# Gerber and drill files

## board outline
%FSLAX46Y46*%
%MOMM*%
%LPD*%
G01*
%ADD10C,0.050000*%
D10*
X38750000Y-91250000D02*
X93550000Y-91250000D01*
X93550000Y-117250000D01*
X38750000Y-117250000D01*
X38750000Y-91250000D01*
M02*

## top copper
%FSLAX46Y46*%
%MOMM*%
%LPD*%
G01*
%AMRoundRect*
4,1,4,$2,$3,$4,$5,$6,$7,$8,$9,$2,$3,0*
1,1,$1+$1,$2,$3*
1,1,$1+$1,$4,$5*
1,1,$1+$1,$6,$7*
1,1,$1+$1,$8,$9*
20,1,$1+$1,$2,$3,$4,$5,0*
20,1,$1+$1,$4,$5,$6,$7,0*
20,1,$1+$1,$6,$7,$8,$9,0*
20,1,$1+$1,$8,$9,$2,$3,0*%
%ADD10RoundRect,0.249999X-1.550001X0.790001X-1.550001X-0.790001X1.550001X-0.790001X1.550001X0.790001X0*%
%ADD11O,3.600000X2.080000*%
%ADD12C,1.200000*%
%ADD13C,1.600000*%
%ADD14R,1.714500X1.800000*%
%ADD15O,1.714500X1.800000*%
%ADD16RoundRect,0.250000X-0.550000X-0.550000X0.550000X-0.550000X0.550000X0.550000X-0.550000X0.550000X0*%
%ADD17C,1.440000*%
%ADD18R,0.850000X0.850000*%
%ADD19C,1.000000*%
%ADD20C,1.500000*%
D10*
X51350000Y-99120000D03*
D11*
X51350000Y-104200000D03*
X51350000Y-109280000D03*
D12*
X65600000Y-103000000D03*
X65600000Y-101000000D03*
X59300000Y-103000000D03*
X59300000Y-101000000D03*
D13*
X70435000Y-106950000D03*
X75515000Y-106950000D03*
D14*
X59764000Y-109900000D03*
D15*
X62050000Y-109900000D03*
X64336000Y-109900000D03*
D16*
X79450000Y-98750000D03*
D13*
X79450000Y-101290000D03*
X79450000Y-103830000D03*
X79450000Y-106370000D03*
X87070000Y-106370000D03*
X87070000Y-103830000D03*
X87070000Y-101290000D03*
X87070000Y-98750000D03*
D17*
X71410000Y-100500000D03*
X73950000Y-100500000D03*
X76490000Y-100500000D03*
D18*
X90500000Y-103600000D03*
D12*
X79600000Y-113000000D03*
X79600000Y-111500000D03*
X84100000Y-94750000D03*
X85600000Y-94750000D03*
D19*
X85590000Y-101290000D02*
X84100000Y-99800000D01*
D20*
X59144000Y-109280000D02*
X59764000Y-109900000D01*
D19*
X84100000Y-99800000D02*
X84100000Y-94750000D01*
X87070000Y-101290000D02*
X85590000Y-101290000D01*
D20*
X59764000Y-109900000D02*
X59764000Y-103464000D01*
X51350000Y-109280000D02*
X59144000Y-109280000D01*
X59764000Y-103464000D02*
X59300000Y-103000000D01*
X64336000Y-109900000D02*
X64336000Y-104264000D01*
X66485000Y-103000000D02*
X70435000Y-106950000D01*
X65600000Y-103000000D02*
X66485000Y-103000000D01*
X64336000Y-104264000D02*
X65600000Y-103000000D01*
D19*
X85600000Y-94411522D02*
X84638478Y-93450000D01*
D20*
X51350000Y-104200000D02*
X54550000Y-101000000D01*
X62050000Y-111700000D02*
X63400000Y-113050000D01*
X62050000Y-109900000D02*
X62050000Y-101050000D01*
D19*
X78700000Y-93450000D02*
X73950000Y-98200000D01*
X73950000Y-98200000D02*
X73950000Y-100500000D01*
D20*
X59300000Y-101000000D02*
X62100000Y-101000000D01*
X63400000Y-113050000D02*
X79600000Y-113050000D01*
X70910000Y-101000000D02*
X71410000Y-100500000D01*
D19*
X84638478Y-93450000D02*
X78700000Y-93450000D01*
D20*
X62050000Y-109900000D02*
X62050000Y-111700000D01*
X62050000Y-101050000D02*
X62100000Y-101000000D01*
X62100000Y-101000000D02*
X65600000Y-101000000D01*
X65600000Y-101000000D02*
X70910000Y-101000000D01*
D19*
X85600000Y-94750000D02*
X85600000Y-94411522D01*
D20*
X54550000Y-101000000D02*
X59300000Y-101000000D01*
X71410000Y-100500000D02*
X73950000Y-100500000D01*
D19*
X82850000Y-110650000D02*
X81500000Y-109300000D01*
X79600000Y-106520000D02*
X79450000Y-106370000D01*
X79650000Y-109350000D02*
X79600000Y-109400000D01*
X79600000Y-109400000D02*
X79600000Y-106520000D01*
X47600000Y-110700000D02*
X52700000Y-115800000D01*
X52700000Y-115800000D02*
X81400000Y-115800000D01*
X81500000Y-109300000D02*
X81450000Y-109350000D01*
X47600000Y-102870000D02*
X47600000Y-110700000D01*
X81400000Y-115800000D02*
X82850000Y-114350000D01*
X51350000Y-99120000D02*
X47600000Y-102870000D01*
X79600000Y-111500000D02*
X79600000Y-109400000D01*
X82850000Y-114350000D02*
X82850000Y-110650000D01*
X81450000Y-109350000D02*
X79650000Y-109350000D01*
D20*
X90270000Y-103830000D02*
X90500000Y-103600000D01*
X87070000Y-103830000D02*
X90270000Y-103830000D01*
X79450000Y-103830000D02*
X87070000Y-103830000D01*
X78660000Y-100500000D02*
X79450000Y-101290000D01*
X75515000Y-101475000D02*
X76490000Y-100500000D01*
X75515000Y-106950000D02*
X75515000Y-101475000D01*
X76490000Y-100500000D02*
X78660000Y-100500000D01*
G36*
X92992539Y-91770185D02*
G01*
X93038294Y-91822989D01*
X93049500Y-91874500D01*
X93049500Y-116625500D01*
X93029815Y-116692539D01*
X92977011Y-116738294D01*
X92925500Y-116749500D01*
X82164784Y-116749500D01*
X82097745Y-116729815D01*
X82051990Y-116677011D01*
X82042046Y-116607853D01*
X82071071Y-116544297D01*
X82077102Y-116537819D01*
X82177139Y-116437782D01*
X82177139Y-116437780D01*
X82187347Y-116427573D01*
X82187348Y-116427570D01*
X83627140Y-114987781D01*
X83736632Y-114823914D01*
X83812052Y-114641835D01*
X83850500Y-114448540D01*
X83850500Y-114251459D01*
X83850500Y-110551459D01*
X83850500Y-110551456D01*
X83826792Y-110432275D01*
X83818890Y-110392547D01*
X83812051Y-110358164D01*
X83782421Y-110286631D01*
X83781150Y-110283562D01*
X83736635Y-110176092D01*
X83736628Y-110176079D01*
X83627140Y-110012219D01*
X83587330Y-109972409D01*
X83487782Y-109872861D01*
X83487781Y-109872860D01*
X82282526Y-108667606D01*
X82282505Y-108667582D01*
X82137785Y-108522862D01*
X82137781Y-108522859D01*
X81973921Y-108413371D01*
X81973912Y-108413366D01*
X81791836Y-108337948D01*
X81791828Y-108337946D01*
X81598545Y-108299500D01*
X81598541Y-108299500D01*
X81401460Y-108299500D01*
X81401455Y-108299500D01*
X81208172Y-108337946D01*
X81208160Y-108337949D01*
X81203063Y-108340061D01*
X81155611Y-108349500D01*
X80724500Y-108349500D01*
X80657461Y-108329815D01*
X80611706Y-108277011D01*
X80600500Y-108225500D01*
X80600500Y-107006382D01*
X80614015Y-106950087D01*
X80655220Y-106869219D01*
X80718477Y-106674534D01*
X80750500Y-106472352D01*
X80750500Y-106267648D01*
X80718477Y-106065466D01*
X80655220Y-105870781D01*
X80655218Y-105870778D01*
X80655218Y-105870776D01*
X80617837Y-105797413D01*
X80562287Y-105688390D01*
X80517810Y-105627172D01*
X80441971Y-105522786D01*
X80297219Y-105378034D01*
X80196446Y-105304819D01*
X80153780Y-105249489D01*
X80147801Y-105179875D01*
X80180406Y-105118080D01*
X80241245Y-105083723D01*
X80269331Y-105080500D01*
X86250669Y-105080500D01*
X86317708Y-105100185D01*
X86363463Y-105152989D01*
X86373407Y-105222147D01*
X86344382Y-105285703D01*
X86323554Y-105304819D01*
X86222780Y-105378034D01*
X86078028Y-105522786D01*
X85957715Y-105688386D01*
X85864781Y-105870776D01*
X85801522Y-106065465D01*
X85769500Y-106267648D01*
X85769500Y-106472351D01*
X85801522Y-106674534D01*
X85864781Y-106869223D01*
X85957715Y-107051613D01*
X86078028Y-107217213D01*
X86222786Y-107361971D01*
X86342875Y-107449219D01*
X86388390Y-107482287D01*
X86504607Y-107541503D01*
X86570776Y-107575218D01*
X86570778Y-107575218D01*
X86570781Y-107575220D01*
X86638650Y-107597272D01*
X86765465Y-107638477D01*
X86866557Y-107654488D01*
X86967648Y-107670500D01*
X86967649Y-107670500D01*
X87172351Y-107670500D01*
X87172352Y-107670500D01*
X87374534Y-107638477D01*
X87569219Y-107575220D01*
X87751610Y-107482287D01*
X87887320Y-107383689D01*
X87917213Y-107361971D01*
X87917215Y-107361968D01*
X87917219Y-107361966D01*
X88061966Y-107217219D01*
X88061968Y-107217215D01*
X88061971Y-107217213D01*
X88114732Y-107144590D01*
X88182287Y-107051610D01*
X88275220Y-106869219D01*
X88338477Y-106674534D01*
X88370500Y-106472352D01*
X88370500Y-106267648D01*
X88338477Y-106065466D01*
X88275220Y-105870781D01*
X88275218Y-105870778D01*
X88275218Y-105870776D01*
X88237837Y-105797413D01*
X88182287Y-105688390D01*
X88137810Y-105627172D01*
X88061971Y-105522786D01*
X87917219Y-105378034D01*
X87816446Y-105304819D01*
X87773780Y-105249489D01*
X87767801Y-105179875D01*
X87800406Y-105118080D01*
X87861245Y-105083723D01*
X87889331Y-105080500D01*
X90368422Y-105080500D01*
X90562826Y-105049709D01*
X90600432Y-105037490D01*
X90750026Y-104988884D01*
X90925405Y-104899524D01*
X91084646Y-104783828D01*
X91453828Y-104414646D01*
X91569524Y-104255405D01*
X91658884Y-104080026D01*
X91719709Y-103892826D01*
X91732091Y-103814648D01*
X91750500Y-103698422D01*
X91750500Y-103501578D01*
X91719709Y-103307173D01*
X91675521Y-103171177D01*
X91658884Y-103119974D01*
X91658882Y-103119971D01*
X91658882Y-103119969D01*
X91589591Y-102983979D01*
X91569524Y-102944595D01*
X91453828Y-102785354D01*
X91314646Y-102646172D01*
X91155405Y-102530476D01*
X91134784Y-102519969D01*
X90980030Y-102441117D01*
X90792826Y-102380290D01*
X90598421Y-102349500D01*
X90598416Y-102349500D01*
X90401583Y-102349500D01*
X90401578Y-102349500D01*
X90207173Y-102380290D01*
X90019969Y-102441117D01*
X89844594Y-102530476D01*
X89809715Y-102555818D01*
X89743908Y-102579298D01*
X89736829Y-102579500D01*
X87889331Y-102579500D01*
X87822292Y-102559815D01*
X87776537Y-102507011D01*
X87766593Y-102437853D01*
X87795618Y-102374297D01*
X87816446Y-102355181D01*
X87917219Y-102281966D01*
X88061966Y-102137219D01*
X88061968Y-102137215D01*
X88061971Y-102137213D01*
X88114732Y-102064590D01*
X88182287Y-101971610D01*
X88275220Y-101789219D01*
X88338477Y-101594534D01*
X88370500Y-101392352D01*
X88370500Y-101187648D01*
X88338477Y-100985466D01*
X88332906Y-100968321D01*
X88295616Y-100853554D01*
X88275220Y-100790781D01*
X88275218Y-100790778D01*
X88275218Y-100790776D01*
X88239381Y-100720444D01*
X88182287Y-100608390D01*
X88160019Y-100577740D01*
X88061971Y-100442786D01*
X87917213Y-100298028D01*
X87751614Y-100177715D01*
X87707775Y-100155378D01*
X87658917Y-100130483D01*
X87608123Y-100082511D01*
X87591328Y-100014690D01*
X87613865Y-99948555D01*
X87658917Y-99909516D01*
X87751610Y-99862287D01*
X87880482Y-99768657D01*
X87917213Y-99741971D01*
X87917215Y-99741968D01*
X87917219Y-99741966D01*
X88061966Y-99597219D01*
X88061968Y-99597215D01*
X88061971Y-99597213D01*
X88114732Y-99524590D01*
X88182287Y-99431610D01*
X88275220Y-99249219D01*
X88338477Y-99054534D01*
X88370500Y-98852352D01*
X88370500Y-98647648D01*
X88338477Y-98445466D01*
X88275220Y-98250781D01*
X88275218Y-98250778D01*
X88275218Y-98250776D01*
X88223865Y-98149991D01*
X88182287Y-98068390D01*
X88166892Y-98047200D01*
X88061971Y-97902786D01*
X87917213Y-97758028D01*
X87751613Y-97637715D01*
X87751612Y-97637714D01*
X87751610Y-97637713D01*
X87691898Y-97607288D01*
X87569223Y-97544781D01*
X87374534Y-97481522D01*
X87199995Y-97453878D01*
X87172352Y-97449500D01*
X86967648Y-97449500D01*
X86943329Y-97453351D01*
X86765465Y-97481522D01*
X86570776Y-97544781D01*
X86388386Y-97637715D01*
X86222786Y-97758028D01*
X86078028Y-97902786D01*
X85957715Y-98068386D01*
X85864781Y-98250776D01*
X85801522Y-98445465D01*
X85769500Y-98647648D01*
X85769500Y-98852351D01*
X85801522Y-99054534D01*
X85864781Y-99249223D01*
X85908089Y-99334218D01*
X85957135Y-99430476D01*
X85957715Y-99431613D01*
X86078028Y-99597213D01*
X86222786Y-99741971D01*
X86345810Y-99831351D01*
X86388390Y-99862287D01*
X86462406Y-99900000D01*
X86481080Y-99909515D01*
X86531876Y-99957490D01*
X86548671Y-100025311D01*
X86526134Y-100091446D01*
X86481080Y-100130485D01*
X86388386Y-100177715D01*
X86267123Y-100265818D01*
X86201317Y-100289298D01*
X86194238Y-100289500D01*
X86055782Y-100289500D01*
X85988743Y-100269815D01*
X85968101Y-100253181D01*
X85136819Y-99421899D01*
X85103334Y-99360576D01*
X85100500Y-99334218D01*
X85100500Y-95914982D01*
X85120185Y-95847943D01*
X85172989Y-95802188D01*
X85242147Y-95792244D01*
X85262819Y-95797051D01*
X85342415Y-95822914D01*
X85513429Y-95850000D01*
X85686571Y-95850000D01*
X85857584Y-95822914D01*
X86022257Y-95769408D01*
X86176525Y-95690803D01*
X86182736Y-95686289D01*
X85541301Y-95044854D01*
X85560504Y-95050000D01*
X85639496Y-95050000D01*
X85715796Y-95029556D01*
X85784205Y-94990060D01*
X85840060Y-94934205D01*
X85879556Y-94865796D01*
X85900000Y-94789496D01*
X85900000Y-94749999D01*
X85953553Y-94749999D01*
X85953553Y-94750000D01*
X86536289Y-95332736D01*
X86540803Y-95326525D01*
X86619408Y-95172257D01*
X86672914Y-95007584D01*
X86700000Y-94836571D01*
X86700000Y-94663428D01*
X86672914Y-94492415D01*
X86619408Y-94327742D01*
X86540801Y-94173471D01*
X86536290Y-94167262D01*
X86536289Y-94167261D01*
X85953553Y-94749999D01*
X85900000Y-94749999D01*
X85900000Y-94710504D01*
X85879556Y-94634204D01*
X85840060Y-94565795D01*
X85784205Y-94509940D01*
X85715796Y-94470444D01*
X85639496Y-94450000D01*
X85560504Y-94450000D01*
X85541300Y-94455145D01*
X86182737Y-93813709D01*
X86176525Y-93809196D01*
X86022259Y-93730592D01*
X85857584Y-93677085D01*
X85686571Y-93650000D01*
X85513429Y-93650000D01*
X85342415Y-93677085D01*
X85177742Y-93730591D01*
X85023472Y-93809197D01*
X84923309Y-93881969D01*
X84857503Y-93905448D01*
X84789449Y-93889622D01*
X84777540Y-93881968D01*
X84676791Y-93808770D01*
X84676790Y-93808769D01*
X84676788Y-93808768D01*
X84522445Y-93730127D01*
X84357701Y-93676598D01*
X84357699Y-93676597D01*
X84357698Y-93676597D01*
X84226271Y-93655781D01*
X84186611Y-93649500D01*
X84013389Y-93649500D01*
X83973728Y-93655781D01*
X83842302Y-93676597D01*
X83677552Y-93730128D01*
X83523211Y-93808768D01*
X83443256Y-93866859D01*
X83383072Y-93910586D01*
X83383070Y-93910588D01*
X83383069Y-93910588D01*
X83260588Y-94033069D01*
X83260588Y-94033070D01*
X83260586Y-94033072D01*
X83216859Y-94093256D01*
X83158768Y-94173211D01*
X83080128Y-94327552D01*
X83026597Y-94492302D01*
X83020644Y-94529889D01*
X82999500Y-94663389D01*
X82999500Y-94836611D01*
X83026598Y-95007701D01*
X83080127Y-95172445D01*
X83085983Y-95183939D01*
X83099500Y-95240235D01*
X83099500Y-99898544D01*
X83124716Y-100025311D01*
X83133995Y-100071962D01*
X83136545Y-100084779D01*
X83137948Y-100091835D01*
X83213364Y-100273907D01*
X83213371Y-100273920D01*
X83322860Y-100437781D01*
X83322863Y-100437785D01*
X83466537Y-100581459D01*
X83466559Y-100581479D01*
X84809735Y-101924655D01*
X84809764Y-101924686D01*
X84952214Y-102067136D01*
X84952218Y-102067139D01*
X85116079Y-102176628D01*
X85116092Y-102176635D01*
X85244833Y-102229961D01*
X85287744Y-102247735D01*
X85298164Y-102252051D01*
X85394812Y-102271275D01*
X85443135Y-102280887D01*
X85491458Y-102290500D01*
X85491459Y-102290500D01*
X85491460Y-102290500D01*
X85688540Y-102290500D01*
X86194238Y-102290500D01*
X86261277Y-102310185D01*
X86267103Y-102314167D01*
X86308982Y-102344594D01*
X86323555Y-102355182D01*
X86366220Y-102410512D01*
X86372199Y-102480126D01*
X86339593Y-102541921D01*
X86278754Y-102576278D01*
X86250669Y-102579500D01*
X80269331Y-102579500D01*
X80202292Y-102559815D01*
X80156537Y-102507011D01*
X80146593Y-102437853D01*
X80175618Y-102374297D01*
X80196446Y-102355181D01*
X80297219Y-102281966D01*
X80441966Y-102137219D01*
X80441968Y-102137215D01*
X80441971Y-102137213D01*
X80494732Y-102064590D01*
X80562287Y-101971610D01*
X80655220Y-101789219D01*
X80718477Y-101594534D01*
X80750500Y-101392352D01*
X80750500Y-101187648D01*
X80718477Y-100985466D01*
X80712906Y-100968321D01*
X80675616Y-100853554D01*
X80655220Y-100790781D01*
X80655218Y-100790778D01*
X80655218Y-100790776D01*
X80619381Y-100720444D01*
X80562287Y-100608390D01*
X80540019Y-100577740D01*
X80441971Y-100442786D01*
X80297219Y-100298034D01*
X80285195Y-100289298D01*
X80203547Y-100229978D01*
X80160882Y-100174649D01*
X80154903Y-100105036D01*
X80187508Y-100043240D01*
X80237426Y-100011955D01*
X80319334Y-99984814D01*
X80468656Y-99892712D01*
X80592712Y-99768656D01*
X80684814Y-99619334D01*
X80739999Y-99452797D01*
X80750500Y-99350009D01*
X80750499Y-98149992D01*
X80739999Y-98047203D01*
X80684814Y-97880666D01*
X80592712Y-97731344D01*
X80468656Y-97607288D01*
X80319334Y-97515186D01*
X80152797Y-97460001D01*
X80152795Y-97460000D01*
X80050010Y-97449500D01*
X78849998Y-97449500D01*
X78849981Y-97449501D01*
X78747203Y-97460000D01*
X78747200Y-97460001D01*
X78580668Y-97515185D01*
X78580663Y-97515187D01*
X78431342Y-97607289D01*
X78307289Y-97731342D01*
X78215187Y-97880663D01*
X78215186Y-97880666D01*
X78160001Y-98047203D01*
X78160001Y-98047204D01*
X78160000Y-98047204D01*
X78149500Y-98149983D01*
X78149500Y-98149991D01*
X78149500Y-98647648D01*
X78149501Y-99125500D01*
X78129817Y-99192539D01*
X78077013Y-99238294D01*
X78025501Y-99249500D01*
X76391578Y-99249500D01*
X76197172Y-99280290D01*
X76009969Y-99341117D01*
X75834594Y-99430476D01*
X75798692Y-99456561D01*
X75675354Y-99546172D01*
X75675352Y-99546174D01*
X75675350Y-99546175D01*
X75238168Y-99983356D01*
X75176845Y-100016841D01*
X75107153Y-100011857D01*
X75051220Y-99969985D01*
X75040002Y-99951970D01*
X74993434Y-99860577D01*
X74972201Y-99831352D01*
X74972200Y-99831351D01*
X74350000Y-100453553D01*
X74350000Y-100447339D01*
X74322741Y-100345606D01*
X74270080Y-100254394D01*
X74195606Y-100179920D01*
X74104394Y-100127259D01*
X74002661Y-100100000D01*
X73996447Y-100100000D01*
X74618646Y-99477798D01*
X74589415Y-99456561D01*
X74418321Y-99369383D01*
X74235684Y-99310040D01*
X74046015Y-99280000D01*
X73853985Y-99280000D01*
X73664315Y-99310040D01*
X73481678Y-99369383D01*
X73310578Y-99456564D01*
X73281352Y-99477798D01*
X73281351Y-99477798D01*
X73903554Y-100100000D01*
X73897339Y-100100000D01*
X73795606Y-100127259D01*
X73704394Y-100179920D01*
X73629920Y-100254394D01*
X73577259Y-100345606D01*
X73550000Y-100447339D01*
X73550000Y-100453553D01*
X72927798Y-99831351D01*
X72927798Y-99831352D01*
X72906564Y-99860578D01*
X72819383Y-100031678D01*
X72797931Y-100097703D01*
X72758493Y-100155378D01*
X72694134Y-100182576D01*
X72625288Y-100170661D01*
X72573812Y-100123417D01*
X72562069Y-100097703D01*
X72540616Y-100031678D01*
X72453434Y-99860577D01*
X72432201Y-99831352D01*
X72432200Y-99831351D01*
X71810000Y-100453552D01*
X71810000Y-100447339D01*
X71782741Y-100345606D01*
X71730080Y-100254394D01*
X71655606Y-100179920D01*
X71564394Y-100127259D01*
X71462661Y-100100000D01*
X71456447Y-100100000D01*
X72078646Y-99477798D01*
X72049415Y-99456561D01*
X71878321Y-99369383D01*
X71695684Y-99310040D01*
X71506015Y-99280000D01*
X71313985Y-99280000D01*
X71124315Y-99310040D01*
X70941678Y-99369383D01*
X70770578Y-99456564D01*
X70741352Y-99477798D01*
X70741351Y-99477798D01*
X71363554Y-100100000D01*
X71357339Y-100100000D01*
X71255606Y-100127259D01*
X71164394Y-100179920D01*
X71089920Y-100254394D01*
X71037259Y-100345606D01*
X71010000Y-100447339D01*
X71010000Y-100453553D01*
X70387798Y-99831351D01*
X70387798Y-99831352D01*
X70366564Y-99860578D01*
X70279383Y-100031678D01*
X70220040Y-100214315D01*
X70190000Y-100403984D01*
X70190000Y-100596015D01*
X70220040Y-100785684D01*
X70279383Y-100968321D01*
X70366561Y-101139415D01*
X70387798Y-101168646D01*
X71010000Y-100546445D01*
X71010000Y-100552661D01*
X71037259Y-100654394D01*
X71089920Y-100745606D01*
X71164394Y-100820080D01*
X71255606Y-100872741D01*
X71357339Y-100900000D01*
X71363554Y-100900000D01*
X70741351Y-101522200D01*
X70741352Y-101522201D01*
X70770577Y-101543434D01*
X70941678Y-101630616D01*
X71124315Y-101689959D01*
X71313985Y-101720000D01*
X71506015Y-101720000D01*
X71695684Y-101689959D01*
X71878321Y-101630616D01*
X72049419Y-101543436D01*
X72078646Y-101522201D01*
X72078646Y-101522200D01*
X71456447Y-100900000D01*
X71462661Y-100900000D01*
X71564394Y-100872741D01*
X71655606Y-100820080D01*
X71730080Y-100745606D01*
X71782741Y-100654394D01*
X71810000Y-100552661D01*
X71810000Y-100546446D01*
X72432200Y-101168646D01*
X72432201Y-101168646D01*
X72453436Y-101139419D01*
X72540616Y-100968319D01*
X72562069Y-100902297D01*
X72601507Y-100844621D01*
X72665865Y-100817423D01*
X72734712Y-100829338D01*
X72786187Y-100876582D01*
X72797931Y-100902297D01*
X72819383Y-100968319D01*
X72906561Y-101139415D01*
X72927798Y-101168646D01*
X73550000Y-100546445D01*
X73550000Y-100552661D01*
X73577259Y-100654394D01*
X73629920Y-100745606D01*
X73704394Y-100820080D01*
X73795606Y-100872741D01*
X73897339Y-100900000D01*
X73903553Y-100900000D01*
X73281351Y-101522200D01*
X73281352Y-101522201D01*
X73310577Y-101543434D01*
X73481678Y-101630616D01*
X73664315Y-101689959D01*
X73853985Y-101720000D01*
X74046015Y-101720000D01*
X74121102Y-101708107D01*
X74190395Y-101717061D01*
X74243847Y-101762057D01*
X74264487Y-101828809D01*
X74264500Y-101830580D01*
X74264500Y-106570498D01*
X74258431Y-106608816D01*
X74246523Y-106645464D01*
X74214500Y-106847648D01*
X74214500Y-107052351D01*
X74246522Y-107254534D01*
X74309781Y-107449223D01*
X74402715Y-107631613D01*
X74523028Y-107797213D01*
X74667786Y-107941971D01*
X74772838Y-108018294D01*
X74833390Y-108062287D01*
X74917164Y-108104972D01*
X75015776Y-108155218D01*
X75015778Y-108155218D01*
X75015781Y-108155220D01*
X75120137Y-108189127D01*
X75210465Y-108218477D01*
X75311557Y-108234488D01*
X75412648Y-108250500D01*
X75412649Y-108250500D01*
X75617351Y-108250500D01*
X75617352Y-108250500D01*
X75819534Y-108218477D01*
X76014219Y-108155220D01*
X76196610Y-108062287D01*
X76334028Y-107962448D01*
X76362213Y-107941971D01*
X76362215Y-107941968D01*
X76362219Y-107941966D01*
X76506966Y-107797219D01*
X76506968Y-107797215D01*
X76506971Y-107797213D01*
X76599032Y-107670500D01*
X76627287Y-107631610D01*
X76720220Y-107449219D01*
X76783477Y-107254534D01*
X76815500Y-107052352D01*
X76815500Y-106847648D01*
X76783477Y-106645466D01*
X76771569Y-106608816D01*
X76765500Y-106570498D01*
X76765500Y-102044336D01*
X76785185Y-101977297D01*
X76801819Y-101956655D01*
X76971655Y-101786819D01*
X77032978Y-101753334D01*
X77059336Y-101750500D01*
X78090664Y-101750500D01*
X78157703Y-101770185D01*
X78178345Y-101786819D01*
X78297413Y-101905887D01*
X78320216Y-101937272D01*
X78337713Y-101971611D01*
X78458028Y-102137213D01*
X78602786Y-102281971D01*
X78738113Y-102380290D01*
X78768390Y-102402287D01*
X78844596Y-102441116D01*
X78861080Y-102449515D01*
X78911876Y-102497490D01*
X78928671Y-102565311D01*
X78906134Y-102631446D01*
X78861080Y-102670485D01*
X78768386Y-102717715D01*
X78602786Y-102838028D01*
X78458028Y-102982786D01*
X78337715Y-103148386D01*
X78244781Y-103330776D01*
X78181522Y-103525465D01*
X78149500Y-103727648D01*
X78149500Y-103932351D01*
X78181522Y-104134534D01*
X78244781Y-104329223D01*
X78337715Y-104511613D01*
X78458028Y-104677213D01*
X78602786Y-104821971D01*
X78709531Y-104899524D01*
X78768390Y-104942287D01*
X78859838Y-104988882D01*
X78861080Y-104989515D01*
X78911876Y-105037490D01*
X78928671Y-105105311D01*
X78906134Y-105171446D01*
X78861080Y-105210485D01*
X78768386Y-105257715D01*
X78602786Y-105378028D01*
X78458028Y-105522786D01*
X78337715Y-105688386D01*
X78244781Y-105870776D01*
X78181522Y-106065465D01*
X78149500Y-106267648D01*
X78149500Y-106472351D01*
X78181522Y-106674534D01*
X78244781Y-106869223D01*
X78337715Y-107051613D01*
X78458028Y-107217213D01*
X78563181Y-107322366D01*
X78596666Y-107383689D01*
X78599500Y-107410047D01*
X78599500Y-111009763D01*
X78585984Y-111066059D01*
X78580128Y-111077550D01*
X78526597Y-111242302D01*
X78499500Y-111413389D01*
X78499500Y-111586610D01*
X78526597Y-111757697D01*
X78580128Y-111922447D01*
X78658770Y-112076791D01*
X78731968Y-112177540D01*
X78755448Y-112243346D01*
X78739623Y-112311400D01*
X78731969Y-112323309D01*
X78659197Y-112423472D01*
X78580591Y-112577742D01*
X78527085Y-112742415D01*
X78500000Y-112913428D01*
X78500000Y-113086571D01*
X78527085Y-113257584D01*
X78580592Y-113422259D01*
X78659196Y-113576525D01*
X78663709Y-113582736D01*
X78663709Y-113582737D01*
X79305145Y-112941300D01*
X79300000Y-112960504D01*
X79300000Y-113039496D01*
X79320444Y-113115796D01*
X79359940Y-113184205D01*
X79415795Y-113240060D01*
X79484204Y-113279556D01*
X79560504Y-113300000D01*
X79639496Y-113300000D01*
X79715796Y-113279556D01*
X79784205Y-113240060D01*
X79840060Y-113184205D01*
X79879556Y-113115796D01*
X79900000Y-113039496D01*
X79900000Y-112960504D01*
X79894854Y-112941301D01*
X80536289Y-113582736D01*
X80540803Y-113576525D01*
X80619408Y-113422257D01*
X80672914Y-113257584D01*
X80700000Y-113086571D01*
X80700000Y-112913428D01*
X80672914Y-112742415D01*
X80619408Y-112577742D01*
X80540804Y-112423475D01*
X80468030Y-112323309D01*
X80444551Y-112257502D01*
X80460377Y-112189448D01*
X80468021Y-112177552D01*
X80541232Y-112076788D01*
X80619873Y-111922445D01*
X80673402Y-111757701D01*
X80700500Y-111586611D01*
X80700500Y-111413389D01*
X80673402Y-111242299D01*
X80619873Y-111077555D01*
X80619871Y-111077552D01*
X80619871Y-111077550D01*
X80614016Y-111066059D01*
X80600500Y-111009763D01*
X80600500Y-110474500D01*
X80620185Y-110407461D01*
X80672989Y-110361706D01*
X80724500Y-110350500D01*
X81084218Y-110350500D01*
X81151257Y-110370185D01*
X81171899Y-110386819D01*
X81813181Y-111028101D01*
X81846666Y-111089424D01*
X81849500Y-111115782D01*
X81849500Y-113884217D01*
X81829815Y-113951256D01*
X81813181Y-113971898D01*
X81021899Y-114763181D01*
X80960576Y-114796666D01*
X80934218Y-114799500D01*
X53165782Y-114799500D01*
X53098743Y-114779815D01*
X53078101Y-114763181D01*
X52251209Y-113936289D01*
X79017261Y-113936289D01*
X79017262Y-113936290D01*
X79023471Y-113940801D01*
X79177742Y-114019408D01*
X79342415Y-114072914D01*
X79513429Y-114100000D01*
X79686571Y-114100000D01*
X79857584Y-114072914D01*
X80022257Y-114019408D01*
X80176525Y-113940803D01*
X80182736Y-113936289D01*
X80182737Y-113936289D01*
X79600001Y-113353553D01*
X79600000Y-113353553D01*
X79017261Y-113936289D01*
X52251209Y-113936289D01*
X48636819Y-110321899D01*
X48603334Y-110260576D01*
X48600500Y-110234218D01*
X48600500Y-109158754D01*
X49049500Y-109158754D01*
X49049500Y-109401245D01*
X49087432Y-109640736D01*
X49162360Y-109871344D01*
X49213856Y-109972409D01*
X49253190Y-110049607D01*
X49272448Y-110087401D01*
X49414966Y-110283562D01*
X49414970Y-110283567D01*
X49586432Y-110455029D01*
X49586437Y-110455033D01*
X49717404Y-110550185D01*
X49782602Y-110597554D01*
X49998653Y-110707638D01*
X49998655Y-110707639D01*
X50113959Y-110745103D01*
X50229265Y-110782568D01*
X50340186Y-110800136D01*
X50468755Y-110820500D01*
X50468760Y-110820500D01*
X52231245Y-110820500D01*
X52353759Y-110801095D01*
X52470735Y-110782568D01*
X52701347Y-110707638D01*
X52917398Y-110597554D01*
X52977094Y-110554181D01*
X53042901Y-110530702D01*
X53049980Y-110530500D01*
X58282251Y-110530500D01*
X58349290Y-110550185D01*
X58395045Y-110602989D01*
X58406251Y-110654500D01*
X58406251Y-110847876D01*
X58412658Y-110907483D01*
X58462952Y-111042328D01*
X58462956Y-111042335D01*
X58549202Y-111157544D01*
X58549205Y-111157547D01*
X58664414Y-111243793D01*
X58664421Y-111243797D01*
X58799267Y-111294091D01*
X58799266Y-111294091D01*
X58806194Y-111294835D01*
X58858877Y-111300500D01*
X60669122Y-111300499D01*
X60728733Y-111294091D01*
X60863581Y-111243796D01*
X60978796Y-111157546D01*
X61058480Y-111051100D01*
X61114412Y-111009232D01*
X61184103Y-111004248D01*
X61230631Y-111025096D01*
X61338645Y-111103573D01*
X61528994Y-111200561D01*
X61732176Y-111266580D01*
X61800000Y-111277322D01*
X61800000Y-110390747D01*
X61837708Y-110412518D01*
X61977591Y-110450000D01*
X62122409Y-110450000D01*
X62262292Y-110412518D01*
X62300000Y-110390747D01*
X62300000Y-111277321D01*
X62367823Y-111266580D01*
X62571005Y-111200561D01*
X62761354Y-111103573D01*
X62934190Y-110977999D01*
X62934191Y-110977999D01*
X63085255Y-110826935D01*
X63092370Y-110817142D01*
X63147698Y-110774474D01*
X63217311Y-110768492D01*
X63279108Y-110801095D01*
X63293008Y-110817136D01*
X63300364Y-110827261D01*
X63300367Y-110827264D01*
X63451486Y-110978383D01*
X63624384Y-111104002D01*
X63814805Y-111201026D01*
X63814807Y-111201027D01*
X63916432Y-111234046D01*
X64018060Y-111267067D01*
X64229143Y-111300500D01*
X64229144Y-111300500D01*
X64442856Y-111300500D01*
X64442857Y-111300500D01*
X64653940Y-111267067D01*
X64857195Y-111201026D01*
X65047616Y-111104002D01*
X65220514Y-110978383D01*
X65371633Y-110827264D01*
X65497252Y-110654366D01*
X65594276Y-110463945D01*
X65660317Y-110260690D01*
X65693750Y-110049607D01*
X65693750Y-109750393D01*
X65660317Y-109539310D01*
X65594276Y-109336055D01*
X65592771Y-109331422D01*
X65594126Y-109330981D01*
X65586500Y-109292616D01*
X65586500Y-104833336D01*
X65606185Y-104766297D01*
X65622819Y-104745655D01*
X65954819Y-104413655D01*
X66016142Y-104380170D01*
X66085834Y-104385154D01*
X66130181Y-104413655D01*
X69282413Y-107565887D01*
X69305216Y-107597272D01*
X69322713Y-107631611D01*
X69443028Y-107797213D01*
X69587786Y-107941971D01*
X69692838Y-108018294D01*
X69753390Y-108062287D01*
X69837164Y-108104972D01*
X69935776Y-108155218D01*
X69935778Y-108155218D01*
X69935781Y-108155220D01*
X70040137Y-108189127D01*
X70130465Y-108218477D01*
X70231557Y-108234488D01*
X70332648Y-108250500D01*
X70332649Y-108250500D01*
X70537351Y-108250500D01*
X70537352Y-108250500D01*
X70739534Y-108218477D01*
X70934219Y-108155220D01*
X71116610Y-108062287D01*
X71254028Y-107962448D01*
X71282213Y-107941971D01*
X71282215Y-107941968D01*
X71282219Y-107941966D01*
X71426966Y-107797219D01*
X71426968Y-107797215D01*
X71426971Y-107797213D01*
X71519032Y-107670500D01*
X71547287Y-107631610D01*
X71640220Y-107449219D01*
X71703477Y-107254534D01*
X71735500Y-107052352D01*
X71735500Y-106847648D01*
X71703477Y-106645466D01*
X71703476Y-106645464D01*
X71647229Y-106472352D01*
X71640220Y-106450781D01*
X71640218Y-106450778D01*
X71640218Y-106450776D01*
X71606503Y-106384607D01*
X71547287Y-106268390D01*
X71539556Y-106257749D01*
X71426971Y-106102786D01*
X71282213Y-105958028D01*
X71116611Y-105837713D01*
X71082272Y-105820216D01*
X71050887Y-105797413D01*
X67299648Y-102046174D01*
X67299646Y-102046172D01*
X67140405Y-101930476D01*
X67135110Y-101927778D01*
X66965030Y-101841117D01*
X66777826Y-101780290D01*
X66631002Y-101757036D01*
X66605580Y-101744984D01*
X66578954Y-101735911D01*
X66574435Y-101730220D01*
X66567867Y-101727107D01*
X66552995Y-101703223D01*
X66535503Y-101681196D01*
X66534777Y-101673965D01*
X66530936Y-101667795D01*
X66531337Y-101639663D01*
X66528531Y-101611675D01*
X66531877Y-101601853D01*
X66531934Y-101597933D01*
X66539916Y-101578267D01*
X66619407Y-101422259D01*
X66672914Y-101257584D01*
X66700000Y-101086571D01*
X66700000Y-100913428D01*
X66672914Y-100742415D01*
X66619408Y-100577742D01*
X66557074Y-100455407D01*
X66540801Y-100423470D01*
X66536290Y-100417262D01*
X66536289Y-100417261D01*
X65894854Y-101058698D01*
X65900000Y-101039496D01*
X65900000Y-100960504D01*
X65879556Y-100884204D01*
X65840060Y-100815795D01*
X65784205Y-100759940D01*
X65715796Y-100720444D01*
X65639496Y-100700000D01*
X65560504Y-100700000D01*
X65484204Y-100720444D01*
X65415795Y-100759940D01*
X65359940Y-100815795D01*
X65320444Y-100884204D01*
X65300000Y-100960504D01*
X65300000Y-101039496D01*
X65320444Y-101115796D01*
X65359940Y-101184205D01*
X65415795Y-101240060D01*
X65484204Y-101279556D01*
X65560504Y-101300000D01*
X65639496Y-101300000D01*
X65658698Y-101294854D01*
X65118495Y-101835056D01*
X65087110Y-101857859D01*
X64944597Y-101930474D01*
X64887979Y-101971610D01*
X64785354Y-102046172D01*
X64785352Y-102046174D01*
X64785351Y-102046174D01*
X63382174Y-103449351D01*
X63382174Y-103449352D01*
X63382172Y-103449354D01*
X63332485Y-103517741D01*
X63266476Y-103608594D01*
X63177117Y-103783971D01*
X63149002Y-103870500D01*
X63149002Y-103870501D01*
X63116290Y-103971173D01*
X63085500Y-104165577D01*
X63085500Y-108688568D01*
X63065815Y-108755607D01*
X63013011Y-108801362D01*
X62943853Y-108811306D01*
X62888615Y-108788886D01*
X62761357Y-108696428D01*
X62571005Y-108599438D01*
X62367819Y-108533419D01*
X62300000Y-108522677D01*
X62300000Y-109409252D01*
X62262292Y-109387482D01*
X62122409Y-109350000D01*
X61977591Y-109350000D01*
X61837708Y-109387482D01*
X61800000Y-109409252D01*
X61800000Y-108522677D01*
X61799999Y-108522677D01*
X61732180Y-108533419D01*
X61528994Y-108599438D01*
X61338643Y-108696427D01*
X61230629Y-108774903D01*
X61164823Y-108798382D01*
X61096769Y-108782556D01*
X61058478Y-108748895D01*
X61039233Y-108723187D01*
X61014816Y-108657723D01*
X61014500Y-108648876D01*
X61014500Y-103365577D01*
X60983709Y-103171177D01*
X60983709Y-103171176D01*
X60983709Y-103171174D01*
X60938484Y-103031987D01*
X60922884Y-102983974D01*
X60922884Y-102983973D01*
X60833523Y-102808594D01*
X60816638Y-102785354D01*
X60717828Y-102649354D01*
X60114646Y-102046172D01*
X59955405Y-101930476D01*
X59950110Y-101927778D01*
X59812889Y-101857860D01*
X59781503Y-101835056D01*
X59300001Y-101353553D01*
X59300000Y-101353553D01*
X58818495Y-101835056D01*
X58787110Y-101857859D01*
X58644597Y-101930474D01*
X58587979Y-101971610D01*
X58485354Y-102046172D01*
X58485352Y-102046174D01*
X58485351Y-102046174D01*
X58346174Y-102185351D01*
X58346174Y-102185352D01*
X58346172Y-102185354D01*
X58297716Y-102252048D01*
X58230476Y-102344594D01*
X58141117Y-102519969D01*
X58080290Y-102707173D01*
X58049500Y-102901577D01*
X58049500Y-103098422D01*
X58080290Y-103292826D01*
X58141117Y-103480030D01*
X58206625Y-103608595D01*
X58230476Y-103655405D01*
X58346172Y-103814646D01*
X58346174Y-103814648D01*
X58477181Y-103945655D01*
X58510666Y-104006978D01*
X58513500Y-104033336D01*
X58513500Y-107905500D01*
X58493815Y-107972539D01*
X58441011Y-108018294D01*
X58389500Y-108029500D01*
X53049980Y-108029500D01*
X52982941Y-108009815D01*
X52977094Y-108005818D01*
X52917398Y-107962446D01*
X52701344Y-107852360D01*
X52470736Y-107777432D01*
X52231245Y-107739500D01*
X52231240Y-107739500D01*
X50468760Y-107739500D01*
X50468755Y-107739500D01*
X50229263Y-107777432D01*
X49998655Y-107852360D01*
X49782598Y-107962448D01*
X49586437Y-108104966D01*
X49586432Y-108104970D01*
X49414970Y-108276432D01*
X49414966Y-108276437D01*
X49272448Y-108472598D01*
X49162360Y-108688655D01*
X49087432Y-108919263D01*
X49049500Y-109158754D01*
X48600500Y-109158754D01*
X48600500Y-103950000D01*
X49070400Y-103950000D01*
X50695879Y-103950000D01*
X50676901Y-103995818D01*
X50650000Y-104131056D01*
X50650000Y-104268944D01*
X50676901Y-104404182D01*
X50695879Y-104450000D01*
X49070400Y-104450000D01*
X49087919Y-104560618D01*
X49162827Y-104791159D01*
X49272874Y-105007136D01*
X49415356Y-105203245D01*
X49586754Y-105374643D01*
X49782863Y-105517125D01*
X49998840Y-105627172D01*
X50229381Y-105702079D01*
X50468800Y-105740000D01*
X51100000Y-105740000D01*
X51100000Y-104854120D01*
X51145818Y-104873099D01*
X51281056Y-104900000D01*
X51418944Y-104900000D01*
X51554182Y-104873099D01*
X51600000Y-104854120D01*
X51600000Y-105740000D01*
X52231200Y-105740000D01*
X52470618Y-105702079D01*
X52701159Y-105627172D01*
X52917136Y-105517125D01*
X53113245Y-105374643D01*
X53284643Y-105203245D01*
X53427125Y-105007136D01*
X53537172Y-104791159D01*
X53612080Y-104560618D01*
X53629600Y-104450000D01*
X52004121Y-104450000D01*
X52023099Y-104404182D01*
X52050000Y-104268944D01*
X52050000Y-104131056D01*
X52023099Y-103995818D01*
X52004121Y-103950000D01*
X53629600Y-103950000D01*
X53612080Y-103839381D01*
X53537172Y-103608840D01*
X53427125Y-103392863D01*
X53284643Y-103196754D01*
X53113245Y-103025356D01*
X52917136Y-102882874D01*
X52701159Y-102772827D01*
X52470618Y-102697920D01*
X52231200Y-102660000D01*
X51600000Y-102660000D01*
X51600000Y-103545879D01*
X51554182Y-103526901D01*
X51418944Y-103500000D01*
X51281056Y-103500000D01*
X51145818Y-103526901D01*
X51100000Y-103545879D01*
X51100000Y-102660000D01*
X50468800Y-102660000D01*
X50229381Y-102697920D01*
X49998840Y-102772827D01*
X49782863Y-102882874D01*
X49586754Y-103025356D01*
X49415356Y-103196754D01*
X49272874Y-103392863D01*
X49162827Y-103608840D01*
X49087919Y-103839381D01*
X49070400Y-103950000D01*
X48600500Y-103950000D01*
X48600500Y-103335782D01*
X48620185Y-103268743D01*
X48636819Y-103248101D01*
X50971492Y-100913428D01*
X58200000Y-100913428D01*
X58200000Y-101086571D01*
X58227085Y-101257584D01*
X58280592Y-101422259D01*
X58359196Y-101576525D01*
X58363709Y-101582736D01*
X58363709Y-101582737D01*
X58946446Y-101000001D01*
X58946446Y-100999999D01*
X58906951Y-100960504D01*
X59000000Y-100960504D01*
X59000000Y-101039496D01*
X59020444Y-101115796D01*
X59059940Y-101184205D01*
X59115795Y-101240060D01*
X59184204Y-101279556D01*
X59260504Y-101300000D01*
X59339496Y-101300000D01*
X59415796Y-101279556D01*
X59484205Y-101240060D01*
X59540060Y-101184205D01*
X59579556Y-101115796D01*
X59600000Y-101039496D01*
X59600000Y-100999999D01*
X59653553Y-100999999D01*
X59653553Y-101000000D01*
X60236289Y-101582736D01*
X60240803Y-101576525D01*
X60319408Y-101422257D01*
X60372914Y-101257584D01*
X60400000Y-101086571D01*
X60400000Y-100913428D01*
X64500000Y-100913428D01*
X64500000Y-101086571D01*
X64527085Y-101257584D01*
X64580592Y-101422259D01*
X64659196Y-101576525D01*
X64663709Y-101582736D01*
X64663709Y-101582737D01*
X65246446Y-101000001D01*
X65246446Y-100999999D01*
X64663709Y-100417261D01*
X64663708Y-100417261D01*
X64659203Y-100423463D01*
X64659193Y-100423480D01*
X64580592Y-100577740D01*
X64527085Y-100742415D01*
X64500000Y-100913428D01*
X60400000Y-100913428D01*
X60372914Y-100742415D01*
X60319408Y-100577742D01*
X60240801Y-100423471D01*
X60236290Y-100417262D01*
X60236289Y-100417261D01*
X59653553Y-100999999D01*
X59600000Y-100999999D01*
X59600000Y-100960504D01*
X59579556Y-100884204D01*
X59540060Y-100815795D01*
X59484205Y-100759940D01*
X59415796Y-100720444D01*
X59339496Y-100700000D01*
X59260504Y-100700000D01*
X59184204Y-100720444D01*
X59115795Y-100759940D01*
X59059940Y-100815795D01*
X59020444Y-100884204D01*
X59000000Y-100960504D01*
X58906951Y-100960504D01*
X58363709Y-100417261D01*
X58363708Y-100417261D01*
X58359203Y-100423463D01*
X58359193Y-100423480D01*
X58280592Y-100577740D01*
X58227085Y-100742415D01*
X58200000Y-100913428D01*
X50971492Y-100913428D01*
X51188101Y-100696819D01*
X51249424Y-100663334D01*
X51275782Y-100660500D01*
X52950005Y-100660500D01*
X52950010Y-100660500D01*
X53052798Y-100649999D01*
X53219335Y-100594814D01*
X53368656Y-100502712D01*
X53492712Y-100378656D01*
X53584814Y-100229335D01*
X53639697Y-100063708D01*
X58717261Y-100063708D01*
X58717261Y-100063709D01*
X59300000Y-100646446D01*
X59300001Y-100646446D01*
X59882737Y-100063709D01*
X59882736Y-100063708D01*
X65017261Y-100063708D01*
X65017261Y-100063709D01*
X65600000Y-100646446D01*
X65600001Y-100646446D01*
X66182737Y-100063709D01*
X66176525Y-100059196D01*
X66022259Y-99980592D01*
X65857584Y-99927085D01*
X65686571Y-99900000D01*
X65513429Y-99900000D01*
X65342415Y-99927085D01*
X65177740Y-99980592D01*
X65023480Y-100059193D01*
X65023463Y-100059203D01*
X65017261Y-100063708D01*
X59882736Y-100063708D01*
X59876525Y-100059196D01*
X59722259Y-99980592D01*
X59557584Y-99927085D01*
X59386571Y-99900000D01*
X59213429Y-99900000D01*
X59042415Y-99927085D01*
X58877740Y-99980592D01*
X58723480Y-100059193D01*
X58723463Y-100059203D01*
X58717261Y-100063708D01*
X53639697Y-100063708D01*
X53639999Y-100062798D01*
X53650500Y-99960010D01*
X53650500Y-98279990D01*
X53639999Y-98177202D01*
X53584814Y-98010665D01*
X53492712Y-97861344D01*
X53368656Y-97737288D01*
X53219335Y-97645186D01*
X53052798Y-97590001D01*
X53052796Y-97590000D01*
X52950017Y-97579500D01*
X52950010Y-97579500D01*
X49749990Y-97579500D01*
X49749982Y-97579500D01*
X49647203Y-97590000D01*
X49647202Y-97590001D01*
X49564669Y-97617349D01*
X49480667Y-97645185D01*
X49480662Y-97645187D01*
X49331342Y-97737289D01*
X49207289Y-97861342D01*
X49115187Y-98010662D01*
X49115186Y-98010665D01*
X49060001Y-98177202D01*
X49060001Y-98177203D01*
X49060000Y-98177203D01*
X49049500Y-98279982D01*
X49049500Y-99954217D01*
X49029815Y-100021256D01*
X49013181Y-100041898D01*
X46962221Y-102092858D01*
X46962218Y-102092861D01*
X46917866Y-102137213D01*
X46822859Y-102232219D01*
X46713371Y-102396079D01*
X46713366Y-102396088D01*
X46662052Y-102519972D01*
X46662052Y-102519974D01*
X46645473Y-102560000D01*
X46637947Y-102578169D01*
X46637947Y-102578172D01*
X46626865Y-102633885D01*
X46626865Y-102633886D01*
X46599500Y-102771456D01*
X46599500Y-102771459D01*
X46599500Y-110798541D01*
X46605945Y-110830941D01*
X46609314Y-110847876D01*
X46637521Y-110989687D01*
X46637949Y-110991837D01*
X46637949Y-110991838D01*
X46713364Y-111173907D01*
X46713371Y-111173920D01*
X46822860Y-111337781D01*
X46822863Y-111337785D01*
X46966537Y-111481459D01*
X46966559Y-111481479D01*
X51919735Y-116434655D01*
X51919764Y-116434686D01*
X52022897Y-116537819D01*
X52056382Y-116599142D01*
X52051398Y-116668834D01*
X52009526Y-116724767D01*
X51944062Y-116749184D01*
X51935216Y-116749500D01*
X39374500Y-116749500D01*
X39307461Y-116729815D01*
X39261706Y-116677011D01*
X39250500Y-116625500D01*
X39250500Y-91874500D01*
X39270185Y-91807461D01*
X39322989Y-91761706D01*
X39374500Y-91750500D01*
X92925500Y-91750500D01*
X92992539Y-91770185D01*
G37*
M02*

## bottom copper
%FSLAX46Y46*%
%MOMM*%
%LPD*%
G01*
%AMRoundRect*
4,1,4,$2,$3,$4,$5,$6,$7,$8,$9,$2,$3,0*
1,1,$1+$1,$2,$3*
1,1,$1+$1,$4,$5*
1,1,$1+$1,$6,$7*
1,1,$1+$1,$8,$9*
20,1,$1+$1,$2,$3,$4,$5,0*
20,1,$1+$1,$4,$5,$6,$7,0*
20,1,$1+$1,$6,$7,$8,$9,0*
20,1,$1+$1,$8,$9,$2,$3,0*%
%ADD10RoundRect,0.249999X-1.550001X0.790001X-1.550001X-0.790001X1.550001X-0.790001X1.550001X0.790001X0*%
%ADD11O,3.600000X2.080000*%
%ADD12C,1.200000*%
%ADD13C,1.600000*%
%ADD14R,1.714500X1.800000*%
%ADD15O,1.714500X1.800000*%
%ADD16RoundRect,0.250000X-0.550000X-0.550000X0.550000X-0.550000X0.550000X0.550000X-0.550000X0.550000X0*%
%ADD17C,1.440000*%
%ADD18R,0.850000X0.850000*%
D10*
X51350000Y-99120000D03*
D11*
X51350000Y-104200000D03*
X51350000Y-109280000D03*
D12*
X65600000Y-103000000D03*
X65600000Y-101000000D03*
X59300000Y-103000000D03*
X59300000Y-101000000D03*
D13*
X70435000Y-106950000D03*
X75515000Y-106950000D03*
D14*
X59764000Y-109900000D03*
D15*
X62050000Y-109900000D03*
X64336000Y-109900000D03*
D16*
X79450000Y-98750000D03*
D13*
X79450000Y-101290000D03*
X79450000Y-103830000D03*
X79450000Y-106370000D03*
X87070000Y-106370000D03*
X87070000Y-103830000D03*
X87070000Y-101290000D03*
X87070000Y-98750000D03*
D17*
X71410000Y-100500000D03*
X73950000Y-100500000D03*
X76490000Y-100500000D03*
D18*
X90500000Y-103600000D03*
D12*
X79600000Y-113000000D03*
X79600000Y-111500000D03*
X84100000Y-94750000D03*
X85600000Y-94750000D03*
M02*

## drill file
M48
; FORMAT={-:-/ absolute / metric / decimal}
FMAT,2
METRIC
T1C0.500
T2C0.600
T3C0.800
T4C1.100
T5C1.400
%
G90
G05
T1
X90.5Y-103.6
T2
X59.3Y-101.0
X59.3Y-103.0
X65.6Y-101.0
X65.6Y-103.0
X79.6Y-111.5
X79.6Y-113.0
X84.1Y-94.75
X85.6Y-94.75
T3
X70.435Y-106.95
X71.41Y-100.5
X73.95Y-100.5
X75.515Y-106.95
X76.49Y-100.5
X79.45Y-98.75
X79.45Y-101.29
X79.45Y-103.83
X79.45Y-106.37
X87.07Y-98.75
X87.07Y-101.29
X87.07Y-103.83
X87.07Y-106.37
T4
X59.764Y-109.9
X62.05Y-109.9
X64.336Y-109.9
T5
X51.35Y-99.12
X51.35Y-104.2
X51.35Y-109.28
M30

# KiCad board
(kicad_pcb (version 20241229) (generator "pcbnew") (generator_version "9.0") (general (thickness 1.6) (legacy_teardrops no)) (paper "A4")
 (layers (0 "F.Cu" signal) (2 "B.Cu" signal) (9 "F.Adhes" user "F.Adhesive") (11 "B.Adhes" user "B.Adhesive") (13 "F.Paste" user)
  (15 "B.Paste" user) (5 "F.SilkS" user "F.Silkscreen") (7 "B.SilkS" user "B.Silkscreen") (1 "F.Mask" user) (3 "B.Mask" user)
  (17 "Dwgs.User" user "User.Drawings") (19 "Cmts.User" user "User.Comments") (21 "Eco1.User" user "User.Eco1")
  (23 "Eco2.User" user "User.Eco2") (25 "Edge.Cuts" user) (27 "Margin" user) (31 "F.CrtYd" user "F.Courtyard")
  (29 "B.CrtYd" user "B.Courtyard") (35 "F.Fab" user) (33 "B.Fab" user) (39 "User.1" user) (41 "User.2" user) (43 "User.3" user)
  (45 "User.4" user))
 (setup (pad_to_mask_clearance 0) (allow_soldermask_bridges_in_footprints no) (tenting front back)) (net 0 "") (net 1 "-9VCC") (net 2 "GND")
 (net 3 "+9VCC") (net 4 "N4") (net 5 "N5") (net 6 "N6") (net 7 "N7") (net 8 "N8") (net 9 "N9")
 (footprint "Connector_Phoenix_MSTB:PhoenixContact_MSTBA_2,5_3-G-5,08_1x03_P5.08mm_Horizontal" (layer "F.Cu") (at 51.35 99.12 -90)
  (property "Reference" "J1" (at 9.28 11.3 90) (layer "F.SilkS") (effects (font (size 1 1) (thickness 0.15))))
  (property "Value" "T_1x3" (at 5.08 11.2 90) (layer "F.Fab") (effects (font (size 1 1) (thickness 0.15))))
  (pad "1" thru_hole roundrect (at 0 0 270) (size 2.08 3.6) (drill 1.4) (layers "*.Cu" "*.Mask") (remove_unused_layers no)
   (roundrect_rratio 0.120192) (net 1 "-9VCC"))
  (pad "2" thru_hole oval (at 5.08 0 270) (size 2.08 3.6) (drill 1.4) (layers "*.Cu" "*.Mask") (remove_unused_layers no) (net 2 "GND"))
  (pad "3" thru_hole oval (at 10.16 0 270) (size 2.08 3.6) (drill 1.4) (layers "*.Cu" "*.Mask") (remove_unused_layers no) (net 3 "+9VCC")))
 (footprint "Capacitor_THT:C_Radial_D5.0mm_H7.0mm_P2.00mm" (layer "F.Cu") (at 65.6 103 90)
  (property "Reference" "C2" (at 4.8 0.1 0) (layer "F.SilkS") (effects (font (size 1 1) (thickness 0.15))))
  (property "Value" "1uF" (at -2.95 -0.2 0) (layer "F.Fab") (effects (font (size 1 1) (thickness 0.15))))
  (pad "1" thru_hole circle (at 0 0 90) (size 1.2 1.2) (drill 0.6) (layers "*.Cu" "*.Mask") (remove_unused_layers no) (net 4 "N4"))
  (pad "2" thru_hole circle (at 2 0 90) (size 1.2 1.2) (drill 0.6) (layers "*.Cu" "*.Mask") (remove_unused_layers no) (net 2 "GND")))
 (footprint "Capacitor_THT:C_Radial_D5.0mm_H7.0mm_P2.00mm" (layer "F.Cu") (at 59.3 103 90)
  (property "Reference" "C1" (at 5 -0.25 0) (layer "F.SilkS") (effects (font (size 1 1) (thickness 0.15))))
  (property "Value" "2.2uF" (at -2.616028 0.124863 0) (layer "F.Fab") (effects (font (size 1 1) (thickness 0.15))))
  (pad "1" thru_hole circle (at 0 0 90) (size 1.2 1.2) (drill 0.6) (layers "*.Cu" "*.Mask") (remove_unused_layers no) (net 3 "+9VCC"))
  (pad "2" thru_hole circle (at 2 0 90) (size 1.2 1.2) (drill 0.6) (layers "*.Cu" "*.Mask") (remove_unused_layers no) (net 2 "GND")))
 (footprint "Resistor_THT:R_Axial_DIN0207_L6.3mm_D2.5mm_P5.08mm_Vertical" (layer "F.Cu") (at 70.435 106.95)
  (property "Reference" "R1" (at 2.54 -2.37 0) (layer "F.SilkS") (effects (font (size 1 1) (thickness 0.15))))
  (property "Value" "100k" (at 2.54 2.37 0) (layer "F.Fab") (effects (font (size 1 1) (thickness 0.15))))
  (pad "1" thru_hole circle (at 0 0) (size 1.6 1.6) (drill 0.8) (layers "*.Cu" "*.Mask") (remove_unused_layers no) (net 4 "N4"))
  (pad "2" thru_hole circle (at 5.08 0) (size 1.6 1.6) (drill 0.8) (layers "*.Cu" "*.Mask") (remove_unused_layers no) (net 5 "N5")))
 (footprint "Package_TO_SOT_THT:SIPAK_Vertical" (layer "F.Cu") (at 59.764 109.9)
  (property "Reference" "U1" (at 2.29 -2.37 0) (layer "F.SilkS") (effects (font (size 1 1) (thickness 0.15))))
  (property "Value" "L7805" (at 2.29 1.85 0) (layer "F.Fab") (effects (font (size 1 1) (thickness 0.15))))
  (pad "1" thru_hole rect (at 0 0) (size 1.7145 1.8) (drill 1.1) (layers "*.Cu" "*.Mask") (remove_unused_layers no) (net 3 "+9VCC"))
  (pad "2" thru_hole oval (at 2.286 0) (size 1.7145 1.8) (drill 1.1) (layers "*.Cu" "*.Mask") (remove_unused_layers no) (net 2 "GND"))
  (pad "3" thru_hole oval (at 4.572 0) (size 1.7145 1.8) (drill 1.1) (layers "*.Cu" "*.Mask") (remove_unused_layers no) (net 4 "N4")))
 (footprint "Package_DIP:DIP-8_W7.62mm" (layer "F.Cu") (at 79.45 98.75)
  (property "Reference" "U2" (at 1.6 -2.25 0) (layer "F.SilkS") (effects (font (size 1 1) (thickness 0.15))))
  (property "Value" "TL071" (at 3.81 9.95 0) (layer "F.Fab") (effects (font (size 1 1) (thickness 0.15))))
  (pad "1" thru_hole roundrect (at 0 0) (size 1.6 1.6) (drill 0.8) (layers "*.Cu" "*.Mask") (remove_unused_layers no)
   (roundrect_rratio 0.15625) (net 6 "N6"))
  (pad "2" thru_hole circle (at 0 2.54) (size 1.6 1.6) (drill 0.8) (layers "*.Cu" "*.Mask") (remove_unused_layers no) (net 5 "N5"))
  (pad "3" thru_hole circle (at 0 5.08) (size 1.6 1.6) (drill 0.8) (layers "*.Cu" "*.Mask") (remove_unused_layers no) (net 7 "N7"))
  (pad "4" thru_hole circle (at 0 7.62) (size 1.6 1.6) (drill 0.8) (layers "*.Cu" "*.Mask") (remove_unused_layers no) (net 1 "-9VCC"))
  (pad "5" thru_hole circle (at 7.62 7.62) (size 1.6 1.6) (drill 0.8) (layers "*.Cu" "*.Mask") (remove_unused_layers no) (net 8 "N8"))
  (pad "6" thru_hole circle (at 7.62 5.08) (size 1.6 1.6) (drill 0.8) (layers "*.Cu" "*.Mask") (remove_unused_layers no) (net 7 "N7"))
  (pad "7" thru_hole circle (at 7.62 2.54) (size 1.6 1.6) (drill 0.8) (layers "*.Cu" "*.Mask") (remove_unused_layers no) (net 3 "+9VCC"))
  (pad "8" thru_hole circle (at 7.62 0) (size 1.6 1.6) (drill 0.8) (layers "*.Cu" "*.Mask") (remove_unused_layers no) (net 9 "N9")))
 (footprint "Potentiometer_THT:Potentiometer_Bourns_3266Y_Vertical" (layer "F.Cu") (at 71.41 100.5 180)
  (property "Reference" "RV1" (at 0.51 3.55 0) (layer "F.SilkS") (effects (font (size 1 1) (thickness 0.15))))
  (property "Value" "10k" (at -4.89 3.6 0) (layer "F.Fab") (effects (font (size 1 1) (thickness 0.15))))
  (pad "1" thru_hole circle (at 0 0 180) (size 1.44 1.44) (drill 0.8) (layers "*.Cu" "*.Mask") (remove_unused_layers no) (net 2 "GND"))
  (pad "2" thru_hole circle (at -2.54 0 180) (size 1.44 1.44) (drill 0.8) (layers "*.Cu" "*.Mask") (remove_unused_layers no) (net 2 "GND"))
  (pad "3" thru_hole circle (at -5.08 0 180) (size 1.44 1.44) (drill 0.8) (layers "*.Cu" "*.Mask") (remove_unused_layers no) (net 5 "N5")))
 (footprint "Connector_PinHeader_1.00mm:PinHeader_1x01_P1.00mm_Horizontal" (layer "F.Cu") (at 90.5 103.6 90)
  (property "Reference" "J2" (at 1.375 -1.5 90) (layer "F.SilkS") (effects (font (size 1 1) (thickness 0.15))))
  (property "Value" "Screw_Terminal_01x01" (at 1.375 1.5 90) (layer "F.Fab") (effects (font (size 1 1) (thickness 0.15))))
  (pad "1" thru_hole rect (at 0 0 90) (size 0.85 0.85) (drill 0.5) (layers "*.Cu" "*.Mask") (remove_unused_layers no) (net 7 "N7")))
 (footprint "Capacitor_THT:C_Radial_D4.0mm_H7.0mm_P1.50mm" (layer "F.Cu") (at 79.6 113 90)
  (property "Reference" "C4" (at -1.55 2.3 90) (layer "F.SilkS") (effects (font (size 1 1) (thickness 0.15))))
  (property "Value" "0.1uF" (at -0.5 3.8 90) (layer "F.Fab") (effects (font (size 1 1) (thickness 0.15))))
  (pad "1" thru_hole circle (at 0 0 90) (size 1.2 1.2) (drill 0.6) (layers "*.Cu" "*.Mask") (remove_unused_layers no) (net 2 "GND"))
  (pad "2" thru_hole circle (at 1.5 0 90) (size 1.2 1.2) (drill 0.6) (layers "*.Cu" "*.Mask") (remove_unused_layers no) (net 1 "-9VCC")))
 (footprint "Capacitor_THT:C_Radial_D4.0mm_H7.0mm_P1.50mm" (layer "F.Cu") (at 84.1 94.75)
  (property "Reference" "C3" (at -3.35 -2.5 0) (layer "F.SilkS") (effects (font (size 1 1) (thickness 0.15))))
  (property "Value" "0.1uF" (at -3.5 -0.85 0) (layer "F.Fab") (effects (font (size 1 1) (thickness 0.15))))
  (pad "1" thru_hole circle (at 0 0) (size 1.2 1.2) (drill 0.6) (layers "*.Cu" "*.Mask") (remove_unused_layers no) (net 3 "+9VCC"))
  (pad "2" thru_hole circle (at 1.5 0) (size 1.2 1.2) (drill 0.6) (layers "*.Cu" "*.Mask") (remove_unused_layers no) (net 2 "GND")))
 (gr_rect (start 38.75 91.25) (end 93.55 117.25) (stroke (width 0.05) (type default)) (fill no) (layer "Edge.Cuts"))
 (segment (start 85.59 101.29) (end 84.1 99.8) (width 1) (layer "F.Cu") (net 3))
 (segment (start 59.144 109.28) (end 59.764 109.9) (width 1.5) (layer "F.Cu") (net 3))
 (segment (start 84.1 99.8) (end 84.1 94.75) (width 1) (layer "F.Cu") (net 3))
 (segment (start 87.07 101.29) (end 85.59 101.29) (width 1) (layer "F.Cu") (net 3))
 (segment (start 59.764 109.9) (end 59.764 103.464) (width 1.5) (layer "F.Cu") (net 3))
 (segment (start 51.35 109.28) (end 59.144 109.28) (width 1.5) (layer "F.Cu") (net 3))
 (segment (start 59.764 103.464) (end 59.3 103) (width 1.5) (layer "F.Cu") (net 3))
 (segment (start 64.336 109.9) (end 64.336 104.264) (width 1.5) (layer "F.Cu") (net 4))
 (segment (start 66.485 103) (end 70.435 106.95) (width 1.5) (layer "F.Cu") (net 4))
 (segment (start 65.6 103) (end 66.485 103) (width 1.5) (layer "F.Cu") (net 4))
 (segment (start 64.336 104.264) (end 65.6 103) (width 1.5) (layer "F.Cu") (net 4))
 (segment (start 85.6 94.411522) (end 84.638478 93.45) (width 1) (layer "F.Cu") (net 2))
 (segment (start 51.35 104.2) (end 54.55 101) (width 1.5) (layer "F.Cu") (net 2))
 (segment (start 62.05 111.7) (end 63.4 113.05) (width 1.5) (layer "F.Cu") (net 2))
 (segment (start 62.05 109.9) (end 62.05 101.05) (width 1.5) (layer "F.Cu") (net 2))
 (segment (start 78.7 93.45) (end 73.95 98.2) (width 1) (layer "F.Cu") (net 2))
 (segment (start 73.95 98.2) (end 73.95 100.5) (width 1) (layer "F.Cu") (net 2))
 (segment (start 59.3 101) (end 62.1 101) (width 1.5) (layer "F.Cu") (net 2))
 (segment (start 63.4 113.05) (end 79.6 113.05) (width 1.5) (layer "F.Cu") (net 2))
 (segment (start 70.91 101) (end 71.41 100.5) (width 1.5) (layer "F.Cu") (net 2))
 (segment (start 84.638478 93.45) (end 78.7 93.45) (width 1) (layer "F.Cu") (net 2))
 (segment (start 62.05 109.9) (end 62.05 111.7) (width 1.5) (layer "F.Cu") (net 2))
 (segment (start 62.05 101.05) (end 62.1 101) (width 1.5) (layer "F.Cu") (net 2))
 (segment (start 62.1 101) (end 65.6 101) (width 1.5) (layer "F.Cu") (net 2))
 (segment (start 65.6 101) (end 70.91 101) (width 1.5) (layer "F.Cu") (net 2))
 (segment (start 85.6 94.75) (end 85.6 94.411522) (width 1) (layer "F.Cu") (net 2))
 (segment (start 54.55 101) (end 59.3 101) (width 1.5) (layer "F.Cu") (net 2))
 (segment (start 71.41 100.5) (end 73.95 100.5) (width 1.5) (layer "F.Cu") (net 2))
 (segment (start 82.85 110.65) (end 81.5 109.3) (width 1) (layer "F.Cu") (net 1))
 (segment (start 79.6 106.52) (end 79.45 106.37) (width 1) (layer "F.Cu") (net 1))
 (segment (start 79.65 109.35) (end 79.6 109.4) (width 1) (layer "F.Cu") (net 1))
 (segment (start 79.6 109.4) (end 79.6 106.52) (width 1) (layer "F.Cu") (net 1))
 (segment (start 47.6 110.7) (end 52.7 115.8) (width 1) (layer "F.Cu") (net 1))
 (segment (start 52.7 115.8) (end 81.4 115.8) (width 1) (layer "F.Cu") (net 1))
 (segment (start 81.5 109.3) (end 81.45 109.35) (width 1) (layer "F.Cu") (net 1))
 (segment (start 47.6 102.87) (end 47.6 110.7) (width 1) (layer "F.Cu") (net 1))
 (segment (start 81.4 115.8) (end 82.85 114.35) (width 1) (layer "F.Cu") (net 1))
 (segment (start 51.35 99.12) (end 47.6 102.87) (width 1) (layer "F.Cu") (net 1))
 (segment (start 79.6 111.5) (end 79.6 109.4) (width 1) (layer "F.Cu") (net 1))
 (segment (start 82.85 114.35) (end 82.85 110.65) (width 1) (layer "F.Cu") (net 1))
 (segment (start 81.45 109.35) (end 79.65 109.35) (width 1) (layer "F.Cu") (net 1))
 (segment (start 90.27 103.83) (end 90.5 103.6) (width 1.5) (layer "F.Cu") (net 7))
 (segment (start 87.07 103.83) (end 90.27 103.83) (width 1.5) (layer "F.Cu") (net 7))
 (segment (start 79.45 103.83) (end 87.07 103.83) (width 1.5) (layer "F.Cu") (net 7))
 (segment (start 78.66 100.5) (end 79.45 101.29) (width 1.5) (layer "F.Cu") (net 5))
 (segment (start 75.515 101.475) (end 76.49 100.5) (width 1.5) (layer "F.Cu") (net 5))
 (segment (start 75.515 106.95) (end 75.515 101.475) (width 1.5) (layer "F.Cu") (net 5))
 (segment (start 76.49 100.5) (end 78.66 100.5) (width 1.5) (layer "F.Cu") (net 5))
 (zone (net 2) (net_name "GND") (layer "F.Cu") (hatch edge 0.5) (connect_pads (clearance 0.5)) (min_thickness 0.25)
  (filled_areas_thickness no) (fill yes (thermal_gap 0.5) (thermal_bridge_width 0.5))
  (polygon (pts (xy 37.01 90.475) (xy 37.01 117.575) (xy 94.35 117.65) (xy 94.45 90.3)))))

